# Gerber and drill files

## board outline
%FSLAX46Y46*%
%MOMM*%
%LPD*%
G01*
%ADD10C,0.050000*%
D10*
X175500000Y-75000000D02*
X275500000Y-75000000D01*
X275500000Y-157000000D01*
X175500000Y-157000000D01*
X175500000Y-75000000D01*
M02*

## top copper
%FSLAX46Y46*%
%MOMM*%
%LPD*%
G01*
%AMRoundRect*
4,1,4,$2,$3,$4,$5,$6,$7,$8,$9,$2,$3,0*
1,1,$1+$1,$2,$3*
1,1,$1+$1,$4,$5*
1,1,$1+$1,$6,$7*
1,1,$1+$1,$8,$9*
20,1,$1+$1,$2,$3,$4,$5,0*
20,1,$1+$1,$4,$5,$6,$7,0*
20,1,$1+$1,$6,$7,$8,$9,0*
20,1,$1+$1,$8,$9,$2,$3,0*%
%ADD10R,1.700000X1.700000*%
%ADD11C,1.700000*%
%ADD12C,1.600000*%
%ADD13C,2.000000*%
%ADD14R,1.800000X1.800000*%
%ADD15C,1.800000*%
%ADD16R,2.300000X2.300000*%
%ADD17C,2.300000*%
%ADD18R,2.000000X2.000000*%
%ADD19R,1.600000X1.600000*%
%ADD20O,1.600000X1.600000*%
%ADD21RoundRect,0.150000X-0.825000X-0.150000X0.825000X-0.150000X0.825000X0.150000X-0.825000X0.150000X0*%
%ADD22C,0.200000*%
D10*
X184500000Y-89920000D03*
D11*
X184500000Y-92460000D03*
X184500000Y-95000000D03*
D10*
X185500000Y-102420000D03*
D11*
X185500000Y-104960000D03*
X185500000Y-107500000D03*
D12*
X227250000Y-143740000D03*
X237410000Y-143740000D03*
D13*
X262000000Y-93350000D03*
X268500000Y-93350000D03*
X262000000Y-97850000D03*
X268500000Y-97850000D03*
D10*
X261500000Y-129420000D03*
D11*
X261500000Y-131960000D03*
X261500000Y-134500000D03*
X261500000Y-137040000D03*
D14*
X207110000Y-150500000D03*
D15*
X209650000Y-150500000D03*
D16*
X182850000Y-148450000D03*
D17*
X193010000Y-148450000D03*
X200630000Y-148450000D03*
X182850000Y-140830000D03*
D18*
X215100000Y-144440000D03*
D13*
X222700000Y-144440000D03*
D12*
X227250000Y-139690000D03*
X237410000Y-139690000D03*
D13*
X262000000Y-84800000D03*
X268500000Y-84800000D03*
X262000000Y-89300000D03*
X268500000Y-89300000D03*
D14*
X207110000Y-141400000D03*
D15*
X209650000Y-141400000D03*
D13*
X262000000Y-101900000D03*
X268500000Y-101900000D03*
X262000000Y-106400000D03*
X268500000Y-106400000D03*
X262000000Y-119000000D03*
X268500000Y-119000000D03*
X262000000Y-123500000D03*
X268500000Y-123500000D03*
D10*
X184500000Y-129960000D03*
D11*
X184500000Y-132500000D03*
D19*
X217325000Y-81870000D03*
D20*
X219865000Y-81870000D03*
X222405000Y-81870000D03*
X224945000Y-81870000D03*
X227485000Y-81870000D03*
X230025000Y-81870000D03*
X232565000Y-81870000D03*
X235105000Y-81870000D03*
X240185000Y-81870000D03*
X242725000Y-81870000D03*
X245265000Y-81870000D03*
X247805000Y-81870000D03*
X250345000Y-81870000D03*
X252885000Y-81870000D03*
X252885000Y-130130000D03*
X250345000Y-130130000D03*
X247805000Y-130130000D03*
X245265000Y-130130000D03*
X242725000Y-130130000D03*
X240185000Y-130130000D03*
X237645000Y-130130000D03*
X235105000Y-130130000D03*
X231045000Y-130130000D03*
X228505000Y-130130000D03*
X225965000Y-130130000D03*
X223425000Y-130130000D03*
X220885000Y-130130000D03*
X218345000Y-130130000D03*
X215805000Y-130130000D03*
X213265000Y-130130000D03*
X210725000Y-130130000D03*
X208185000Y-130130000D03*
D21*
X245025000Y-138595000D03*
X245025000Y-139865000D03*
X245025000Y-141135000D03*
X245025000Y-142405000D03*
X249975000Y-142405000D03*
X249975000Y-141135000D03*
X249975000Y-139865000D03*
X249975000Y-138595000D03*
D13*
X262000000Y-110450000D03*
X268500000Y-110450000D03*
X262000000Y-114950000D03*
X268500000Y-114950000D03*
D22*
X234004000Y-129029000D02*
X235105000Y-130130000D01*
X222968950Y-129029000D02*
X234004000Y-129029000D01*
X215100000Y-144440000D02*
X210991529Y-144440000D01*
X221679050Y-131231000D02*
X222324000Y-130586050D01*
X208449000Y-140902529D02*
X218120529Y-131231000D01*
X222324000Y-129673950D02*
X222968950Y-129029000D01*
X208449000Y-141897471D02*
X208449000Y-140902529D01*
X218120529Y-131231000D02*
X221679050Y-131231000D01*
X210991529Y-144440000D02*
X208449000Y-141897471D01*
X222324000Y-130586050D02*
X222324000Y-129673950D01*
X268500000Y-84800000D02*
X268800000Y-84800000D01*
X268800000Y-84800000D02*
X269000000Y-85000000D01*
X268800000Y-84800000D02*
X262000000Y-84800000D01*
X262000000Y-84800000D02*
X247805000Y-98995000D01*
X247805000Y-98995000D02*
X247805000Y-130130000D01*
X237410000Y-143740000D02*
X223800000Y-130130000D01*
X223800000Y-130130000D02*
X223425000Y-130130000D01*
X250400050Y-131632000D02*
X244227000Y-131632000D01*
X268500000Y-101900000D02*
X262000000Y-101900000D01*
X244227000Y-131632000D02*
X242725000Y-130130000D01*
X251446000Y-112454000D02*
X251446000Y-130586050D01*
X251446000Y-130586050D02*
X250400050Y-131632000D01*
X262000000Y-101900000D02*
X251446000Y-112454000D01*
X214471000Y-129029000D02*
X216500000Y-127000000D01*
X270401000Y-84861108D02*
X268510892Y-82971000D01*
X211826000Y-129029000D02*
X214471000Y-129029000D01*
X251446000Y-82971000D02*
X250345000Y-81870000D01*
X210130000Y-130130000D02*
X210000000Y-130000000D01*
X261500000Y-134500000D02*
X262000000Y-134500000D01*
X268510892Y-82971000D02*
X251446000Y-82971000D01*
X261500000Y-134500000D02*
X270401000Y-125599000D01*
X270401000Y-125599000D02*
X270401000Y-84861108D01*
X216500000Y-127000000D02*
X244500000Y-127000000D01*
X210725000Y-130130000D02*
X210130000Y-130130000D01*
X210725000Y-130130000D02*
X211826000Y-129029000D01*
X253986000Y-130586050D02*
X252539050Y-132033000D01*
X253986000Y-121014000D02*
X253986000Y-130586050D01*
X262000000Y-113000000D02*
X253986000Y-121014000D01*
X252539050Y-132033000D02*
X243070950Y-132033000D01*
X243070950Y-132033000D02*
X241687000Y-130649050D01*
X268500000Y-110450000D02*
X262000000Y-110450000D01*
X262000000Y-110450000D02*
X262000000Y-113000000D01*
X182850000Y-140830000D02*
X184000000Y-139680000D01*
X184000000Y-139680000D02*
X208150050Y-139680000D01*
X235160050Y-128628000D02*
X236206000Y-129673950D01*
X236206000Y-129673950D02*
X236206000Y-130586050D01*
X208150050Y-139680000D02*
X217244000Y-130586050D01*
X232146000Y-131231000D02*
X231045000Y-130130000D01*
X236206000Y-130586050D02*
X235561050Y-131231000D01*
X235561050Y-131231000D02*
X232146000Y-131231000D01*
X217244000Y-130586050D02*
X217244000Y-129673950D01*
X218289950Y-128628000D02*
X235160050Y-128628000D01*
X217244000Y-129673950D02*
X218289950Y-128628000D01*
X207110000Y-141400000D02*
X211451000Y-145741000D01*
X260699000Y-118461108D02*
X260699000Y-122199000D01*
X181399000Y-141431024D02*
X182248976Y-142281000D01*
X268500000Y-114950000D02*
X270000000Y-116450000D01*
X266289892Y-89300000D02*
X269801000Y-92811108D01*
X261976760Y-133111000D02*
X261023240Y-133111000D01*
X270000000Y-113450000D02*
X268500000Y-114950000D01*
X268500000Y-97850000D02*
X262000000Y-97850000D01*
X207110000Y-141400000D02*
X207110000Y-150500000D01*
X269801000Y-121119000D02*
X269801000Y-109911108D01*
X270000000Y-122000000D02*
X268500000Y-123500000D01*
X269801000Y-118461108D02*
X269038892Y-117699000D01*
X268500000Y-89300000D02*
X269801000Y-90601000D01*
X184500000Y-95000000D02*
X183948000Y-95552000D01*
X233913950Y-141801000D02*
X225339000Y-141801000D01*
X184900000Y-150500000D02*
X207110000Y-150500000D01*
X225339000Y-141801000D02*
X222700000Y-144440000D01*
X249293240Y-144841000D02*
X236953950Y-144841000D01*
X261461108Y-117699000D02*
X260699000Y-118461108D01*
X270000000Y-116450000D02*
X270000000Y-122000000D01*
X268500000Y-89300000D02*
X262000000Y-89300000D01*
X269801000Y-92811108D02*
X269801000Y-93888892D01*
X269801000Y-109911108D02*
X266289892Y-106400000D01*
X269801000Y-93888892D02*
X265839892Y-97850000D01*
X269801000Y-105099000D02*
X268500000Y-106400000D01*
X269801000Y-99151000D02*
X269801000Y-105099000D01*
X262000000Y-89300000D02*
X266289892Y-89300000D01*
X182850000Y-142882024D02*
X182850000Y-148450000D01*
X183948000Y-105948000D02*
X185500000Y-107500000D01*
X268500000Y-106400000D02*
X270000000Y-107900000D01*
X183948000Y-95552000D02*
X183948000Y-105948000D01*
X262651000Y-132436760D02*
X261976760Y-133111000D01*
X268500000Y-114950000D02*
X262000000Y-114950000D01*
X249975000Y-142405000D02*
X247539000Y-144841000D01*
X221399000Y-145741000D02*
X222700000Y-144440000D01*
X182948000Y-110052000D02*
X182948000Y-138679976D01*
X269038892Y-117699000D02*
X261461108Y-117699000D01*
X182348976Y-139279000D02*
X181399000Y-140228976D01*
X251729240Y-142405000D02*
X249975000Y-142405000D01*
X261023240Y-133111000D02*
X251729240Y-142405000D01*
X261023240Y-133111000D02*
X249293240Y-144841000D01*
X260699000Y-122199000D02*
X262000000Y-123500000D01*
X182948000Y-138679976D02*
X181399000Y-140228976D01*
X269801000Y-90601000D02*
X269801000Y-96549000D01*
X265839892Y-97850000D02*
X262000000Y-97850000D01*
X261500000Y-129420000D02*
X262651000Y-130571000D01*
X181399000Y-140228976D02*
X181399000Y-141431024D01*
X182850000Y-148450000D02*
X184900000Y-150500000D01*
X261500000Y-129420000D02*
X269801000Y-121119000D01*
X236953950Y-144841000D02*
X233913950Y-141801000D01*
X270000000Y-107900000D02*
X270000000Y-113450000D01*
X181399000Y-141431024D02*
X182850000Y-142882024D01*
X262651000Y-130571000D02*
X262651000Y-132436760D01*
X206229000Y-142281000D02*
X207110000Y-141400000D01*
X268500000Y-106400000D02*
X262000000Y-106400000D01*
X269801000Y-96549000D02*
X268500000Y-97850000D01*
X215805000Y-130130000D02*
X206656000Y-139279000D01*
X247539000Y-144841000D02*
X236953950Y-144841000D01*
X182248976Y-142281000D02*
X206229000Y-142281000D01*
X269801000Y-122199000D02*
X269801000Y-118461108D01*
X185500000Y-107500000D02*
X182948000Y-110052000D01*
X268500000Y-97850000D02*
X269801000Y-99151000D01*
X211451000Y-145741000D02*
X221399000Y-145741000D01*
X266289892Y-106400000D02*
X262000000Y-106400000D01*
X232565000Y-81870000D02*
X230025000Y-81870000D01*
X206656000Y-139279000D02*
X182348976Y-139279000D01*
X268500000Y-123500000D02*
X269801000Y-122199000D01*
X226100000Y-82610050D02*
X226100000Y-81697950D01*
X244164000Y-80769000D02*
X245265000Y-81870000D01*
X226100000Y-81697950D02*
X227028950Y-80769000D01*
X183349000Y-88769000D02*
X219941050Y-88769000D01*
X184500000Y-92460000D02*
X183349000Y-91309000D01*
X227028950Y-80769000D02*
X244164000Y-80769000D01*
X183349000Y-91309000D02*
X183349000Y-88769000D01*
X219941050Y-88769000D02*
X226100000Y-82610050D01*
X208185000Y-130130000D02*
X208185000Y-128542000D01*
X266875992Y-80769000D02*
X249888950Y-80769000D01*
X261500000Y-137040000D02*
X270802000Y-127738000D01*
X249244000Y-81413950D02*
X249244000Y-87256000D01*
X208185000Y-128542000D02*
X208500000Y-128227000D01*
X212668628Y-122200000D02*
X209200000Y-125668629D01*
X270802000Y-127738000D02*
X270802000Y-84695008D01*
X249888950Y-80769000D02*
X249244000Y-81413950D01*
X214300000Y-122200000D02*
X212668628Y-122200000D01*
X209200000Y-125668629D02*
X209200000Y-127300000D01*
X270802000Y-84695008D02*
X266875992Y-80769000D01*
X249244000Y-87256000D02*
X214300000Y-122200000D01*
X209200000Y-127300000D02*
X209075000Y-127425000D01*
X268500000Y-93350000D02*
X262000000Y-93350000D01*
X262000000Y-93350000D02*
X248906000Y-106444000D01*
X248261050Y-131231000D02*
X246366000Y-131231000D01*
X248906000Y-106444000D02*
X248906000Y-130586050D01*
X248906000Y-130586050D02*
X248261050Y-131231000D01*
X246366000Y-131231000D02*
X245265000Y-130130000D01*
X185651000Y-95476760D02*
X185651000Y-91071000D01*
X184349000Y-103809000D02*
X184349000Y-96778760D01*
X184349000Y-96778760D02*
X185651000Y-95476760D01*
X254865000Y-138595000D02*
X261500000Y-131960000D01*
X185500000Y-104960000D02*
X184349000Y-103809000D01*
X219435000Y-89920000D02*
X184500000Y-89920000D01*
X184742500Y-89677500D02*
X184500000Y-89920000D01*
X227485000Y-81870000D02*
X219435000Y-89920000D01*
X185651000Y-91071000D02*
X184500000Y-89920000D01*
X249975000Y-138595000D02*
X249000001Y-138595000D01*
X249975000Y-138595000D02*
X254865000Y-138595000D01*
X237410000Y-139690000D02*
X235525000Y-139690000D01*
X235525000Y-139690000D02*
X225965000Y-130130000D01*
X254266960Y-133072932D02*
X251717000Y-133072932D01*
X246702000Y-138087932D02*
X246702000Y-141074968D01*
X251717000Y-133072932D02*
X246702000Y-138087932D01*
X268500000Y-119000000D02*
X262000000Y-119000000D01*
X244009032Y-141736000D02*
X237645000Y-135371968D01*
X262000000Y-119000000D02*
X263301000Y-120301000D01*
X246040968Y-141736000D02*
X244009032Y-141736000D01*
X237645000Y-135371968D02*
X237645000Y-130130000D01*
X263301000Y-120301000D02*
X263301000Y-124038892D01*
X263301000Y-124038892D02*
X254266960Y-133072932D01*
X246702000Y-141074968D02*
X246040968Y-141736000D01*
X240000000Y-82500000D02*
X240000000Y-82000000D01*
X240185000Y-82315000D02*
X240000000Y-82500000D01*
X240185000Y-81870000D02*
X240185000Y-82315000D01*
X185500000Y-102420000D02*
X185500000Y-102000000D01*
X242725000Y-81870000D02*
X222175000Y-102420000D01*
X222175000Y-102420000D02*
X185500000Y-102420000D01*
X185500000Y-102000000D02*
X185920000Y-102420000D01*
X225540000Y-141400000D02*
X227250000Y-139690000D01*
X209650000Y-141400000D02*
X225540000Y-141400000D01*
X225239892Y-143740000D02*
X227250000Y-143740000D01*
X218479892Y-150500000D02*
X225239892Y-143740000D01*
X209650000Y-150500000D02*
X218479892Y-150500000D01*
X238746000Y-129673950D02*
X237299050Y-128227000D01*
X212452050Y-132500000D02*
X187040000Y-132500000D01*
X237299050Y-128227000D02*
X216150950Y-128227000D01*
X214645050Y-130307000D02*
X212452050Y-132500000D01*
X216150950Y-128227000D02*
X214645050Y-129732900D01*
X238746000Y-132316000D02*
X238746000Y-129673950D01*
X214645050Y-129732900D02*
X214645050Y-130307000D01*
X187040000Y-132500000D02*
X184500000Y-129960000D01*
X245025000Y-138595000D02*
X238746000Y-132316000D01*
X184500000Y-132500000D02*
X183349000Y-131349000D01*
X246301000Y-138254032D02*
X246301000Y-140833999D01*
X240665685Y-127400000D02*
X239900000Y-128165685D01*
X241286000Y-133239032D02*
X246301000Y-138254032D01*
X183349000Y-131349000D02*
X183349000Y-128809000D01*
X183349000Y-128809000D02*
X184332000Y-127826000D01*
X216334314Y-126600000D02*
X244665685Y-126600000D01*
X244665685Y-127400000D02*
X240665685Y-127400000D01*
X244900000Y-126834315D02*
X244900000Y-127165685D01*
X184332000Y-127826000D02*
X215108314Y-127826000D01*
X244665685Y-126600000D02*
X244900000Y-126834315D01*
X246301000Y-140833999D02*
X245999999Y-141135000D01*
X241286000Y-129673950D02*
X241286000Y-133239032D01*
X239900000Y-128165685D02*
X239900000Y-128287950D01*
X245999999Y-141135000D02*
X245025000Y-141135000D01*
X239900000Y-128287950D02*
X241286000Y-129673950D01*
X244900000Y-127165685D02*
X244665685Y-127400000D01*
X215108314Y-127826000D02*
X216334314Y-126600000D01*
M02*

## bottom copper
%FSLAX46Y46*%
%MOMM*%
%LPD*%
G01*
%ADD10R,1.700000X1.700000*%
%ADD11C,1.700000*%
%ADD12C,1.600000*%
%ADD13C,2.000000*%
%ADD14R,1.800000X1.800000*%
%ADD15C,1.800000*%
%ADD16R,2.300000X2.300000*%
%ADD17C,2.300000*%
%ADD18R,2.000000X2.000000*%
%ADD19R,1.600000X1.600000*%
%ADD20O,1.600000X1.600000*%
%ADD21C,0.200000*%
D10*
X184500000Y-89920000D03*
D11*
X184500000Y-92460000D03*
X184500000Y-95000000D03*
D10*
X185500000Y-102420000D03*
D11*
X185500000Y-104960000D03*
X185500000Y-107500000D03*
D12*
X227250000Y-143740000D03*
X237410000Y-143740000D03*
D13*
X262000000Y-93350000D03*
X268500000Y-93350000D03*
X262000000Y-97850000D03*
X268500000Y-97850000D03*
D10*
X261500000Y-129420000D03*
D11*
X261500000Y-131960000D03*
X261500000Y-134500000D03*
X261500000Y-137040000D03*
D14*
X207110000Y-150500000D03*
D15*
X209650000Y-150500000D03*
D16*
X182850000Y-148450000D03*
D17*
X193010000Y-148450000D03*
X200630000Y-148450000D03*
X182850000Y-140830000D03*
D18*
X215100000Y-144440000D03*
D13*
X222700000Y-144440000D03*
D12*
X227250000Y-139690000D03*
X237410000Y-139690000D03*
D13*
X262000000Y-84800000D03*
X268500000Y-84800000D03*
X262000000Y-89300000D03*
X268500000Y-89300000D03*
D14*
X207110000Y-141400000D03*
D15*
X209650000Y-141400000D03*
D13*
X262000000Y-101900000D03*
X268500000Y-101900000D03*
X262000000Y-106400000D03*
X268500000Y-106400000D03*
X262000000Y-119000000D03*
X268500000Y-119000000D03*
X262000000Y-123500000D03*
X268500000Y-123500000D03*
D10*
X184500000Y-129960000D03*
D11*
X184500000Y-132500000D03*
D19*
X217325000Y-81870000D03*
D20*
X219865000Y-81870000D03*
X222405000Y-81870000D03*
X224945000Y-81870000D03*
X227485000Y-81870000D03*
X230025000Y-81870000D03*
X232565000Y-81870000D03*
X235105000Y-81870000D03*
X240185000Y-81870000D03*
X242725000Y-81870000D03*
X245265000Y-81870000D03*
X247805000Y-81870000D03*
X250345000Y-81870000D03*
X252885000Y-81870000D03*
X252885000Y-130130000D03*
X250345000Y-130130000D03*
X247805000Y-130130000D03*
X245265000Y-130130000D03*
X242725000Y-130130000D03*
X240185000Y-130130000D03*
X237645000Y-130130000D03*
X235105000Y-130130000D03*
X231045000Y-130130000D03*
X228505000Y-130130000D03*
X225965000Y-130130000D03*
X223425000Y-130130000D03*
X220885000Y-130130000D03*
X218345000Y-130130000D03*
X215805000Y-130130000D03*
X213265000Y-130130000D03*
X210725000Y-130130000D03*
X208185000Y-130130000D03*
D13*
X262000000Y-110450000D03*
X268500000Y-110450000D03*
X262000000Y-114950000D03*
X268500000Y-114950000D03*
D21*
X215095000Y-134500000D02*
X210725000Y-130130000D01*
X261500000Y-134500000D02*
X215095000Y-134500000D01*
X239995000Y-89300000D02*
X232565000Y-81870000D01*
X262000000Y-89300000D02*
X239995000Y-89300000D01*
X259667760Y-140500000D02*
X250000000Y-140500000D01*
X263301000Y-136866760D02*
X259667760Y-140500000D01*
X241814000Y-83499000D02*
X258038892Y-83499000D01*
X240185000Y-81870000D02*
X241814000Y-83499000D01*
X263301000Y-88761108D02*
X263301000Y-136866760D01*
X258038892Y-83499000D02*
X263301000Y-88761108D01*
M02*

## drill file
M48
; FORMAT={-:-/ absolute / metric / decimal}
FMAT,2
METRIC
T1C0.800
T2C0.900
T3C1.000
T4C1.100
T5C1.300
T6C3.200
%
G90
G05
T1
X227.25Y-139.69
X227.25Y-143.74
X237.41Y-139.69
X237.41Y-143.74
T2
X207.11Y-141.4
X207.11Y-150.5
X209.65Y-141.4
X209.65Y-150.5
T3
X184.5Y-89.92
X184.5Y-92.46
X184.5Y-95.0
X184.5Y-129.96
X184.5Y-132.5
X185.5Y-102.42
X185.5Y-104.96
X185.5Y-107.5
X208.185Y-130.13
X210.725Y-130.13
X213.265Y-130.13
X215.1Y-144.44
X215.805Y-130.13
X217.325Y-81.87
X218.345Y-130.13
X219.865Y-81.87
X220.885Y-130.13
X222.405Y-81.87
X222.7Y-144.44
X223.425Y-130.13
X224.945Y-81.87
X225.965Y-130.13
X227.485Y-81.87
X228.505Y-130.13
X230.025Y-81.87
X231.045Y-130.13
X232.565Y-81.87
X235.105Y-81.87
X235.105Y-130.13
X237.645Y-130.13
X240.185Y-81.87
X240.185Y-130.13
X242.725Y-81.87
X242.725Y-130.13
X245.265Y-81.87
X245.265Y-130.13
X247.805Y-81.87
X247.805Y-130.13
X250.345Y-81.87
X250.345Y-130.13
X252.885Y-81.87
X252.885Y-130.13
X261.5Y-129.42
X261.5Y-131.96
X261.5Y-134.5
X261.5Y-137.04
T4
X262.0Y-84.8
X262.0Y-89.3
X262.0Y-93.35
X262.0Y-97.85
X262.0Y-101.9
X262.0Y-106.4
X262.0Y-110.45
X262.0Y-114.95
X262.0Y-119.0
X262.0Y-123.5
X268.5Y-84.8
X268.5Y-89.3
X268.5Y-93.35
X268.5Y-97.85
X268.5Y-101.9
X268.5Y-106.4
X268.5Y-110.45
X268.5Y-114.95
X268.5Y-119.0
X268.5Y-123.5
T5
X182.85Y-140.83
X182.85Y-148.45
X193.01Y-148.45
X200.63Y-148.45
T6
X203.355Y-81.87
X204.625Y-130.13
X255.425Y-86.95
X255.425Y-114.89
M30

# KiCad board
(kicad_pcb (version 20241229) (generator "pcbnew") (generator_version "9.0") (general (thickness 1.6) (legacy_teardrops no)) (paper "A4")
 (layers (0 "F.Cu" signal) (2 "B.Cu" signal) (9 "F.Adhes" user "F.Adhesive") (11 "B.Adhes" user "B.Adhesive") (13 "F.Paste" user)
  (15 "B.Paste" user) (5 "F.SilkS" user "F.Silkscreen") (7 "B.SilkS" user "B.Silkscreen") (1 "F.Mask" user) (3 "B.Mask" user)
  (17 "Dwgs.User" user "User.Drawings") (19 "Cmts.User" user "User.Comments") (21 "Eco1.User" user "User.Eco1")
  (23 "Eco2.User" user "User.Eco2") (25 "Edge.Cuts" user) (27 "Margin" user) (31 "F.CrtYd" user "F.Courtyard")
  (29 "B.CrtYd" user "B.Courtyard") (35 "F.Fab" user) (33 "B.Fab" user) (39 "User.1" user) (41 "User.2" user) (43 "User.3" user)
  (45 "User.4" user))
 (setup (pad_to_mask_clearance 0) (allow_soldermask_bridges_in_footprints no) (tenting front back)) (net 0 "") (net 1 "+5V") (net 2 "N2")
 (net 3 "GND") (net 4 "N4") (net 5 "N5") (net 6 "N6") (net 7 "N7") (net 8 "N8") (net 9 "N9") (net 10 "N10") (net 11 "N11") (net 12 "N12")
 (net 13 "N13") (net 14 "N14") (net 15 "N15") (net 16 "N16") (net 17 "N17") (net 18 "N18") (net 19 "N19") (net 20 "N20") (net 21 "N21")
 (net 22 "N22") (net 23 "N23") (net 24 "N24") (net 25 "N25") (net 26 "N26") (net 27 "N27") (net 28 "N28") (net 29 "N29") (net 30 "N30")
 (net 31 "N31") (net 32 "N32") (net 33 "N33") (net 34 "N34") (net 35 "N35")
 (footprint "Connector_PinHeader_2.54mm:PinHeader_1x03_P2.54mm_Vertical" (layer "F.Cu") (at 184.5 89.92)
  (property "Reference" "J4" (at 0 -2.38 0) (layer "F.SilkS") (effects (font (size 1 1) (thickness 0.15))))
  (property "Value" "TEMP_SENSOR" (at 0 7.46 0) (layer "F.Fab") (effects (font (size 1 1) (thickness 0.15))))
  (pad "1" thru_hole rect (at 0 0) (size 1.7 1.7) (drill 1) (layers "*.Cu" "*.Mask") (remove_unused_layers no) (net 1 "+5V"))
  (pad "2" thru_hole circle (at 0 2.54) (size 1.7 1.7) (drill 1) (layers "*.Cu" "*.Mask") (remove_unused_layers no) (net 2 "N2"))
  (pad "3" thru_hole circle (at 0 5.08) (size 1.7 1.7) (drill 1) (layers "*.Cu" "*.Mask") (remove_unused_layers no) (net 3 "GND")))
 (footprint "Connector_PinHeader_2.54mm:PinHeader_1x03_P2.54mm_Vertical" (layer "F.Cu") (at 185.5 102.42)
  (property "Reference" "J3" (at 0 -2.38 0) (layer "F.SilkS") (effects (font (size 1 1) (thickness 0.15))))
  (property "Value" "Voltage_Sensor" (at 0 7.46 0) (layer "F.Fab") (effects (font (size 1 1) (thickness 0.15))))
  (pad "1" thru_hole rect (at 0 0) (size 1.7 1.7) (drill 1) (layers "*.Cu" "*.Mask") (remove_unused_layers no) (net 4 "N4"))
  (pad "2" thru_hole circle (at 0 2.54) (size 1.7 1.7) (drill 1) (layers "*.Cu" "*.Mask") (remove_unused_layers no) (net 1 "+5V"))
  (pad "3" thru_hole circle (at 0 5.08) (size 1.7 1.7) (drill 1) (layers "*.Cu" "*.Mask") (remove_unused_layers no) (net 3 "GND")))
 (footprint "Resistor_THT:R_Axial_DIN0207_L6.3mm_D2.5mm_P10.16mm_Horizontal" (layer "F.Cu") (at 227.25 143.74)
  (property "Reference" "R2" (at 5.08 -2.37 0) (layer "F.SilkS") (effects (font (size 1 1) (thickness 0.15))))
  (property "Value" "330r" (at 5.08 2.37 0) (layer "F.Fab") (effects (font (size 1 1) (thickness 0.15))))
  (pad "1" thru_hole circle (at 0 0) (size 1.6 1.6) (drill 0.8) (layers "*.Cu" "*.Mask") (remove_unused_layers no) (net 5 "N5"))
  (pad "2" thru_hole circle (at 10.16 0) (size 1.6 1.6) (drill 0.8) (layers "*.Cu" "*.Mask") (remove_unused_layers no) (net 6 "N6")))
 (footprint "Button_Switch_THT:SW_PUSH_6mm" (layer "F.Cu") (at 262 93.35)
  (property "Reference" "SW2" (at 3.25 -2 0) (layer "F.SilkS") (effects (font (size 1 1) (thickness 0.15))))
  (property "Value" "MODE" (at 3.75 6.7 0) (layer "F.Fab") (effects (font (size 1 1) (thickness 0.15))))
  (pad "1" thru_hole circle (at 0 0 90) (size 2 2) (drill 1.1) (layers "*.Cu" "*.Mask") (remove_unused_layers no) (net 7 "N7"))
  (pad "1" thru_hole circle (at 6.5 0 90) (size 2 2) (drill 1.1) (layers "*.Cu" "*.Mask") (remove_unused_layers no) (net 7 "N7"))
  (pad "2" thru_hole circle (at 0 4.5 90) (size 2 2) (drill 1.1) (layers "*.Cu" "*.Mask") (remove_unused_layers no) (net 3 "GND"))
  (pad "2" thru_hole circle (at 6.5 4.5 90) (size 2 2) (drill 1.1) (layers "*.Cu" "*.Mask") (remove_unused_layers no) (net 3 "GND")))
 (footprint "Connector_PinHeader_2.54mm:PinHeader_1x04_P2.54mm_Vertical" (layer "F.Cu") (at 261.5 129.42)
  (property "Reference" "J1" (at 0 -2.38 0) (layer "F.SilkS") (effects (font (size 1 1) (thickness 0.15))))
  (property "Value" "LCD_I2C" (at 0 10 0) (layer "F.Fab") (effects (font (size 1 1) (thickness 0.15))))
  (pad "1" thru_hole rect (at 0 0) (size 1.7 1.7) (drill 1) (layers "*.Cu" "*.Mask") (remove_unused_layers no) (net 3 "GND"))
  (pad "2" thru_hole circle (at 0 2.54) (size 1.7 1.7) (drill 1) (layers "*.Cu" "*.Mask") (remove_unused_layers no) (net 1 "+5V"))
  (pad "3" thru_hole circle (at 0 5.08) (size 1.7 1.7) (drill 1) (layers "*.Cu" "*.Mask") (remove_unused_layers no) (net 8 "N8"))
  (pad "4" thru_hole circle (at 0 7.62) (size 1.7 1.7) (drill 1) (layers "*.Cu" "*.Mask") (remove_unused_layers no) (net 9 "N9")))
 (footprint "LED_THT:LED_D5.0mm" (layer "F.Cu") (at 207.11 150.5)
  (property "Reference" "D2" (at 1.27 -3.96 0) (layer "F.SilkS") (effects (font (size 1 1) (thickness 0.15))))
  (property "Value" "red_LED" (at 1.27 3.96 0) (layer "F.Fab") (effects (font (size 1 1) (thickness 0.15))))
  (pad "1" thru_hole rect (at 0 0) (size 1.8 1.8) (drill 0.9) (layers "*.Cu" "*.Mask") (remove_unused_layers no) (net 3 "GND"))
  (pad "2" thru_hole circle (at 2.54 0) (size 1.8 1.8) (drill 0.9) (layers "*.Cu" "*.Mask") (remove_unused_layers no) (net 5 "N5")))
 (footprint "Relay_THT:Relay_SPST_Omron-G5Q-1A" (layer "F.Cu") (at 182.85 148.45)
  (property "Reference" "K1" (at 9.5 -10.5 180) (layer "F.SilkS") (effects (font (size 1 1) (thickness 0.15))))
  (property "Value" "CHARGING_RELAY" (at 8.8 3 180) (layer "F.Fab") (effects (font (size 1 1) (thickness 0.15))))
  (pad "1" thru_hole rect (at 0 0 180) (size 2.3 2.3) (drill 1.3) (layers "*.Cu" "*.Mask") (remove_unused_layers no) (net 3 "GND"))
  (pad "2" thru_hole circle (at 10.16 0 180) (size 2.3 2.3) (drill 1.3) (layers "*.Cu" "*.Mask") (remove_unused_layers no) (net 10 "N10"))
  (pad "3" thru_hole circle (at 17.78 0 180) (size 2.3 2.3) (drill 1.3) (layers "*.Cu" "*.Mask") (remove_unused_layers no) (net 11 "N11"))
  (pad "5" thru_hole circle (at 0 -7.62 180) (size 2.3 2.3) (drill 1.3) (layers "*.Cu" "*.Mask") (remove_unused_layers no) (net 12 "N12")))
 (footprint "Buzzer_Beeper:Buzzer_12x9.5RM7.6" (layer "F.Cu") (at 215.1 144.44)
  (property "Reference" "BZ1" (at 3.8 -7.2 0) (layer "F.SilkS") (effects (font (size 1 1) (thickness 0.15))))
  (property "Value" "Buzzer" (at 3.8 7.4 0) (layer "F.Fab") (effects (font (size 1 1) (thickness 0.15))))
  (pad "1" thru_hole rect (at 0 0) (size 2 2) (drill 1) (layers "*.Cu" "*.Mask") (remove_unused_layers no) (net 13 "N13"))
  (pad "2" thru_hole circle (at 7.6 0) (size 2 2) (drill 1) (layers "*.Cu" "*.Mask") (remove_unused_layers no) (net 3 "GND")))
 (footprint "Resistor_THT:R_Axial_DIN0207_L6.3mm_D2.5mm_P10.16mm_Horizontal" (layer "F.Cu") (at 227.25 139.69)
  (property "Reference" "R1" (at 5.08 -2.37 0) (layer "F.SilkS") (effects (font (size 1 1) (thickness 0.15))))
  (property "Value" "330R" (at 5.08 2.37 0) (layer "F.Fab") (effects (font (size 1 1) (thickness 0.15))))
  (pad "1" thru_hole circle (at 0 0) (size 1.6 1.6) (drill 0.8) (layers "*.Cu" "*.Mask") (remove_unused_layers no) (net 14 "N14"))
  (pad "2" thru_hole circle (at 10.16 0) (size 1.6 1.6) (drill 0.8) (layers "*.Cu" "*.Mask") (remove_unused_layers no) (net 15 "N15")))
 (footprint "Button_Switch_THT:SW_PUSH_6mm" (layer "F.Cu") (at 262 84.8)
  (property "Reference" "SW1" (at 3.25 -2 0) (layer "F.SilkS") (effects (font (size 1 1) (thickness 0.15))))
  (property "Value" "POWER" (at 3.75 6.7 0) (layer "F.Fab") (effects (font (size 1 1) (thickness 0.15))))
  (pad "1" thru_hole circle (at 0 0 90) (size 2 2) (drill 1.1) (layers "*.Cu" "*.Mask") (remove_unused_layers no) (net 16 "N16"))
  (pad "1" thru_hole circle (at 6.5 0 90) (size 2 2) (drill 1.1) (layers "*.Cu" "*.Mask") (remove_unused_layers no) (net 16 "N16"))
  (pad "2" thru_hole circle (at 0 4.5 90) (size 2 2) (drill 1.1) (layers "*.Cu" "*.Mask") (remove_unused_layers no) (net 3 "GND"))
  (pad "2" thru_hole circle (at 6.5 4.5 90) (size 2 2) (drill 1.1) (layers "*.Cu" "*.Mask") (remove_unused_layers no) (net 3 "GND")))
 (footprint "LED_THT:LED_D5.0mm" (layer "F.Cu") (at 207.11 141.4)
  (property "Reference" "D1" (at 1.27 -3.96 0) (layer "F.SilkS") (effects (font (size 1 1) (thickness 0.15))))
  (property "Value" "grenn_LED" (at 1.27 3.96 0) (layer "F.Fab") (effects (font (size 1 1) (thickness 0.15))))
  (pad "1" thru_hole rect (at 0 0) (size 1.8 1.8) (drill 0.9) (layers "*.Cu" "*.Mask") (remove_unused_layers no) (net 3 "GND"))
  (pad "2" thru_hole circle (at 2.54 0) (size 1.8 1.8) (drill 0.9) (layers "*.Cu" "*.Mask") (remove_unused_layers no) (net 14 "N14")))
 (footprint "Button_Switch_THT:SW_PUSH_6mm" (layer "F.Cu") (at 262 101.9)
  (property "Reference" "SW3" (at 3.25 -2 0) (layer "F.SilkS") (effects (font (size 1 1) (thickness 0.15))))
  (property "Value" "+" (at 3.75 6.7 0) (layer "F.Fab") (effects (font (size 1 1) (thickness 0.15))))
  (pad "1" thru_hole circle (at 0 0 90) (size 2 2) (drill 1.1) (layers "*.Cu" "*.Mask") (remove_unused_layers no) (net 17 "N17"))
  (pad "1" thru_hole circle (at 6.5 0 90) (size 2 2) (drill 1.1) (layers "*.Cu" "*.Mask") (remove_unused_layers no) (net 17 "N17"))
  (pad "2" thru_hole circle (at 0 4.5 90) (size 2 2) (drill 1.1) (layers "*.Cu" "*.Mask") (remove_unused_layers no) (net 3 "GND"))
  (pad "2" thru_hole circle (at 6.5 4.5 90) (size 2 2) (drill 1.1) (layers "*.Cu" "*.Mask") (remove_unused_layers no) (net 3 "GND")))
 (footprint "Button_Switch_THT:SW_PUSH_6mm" (layer "F.Cu") (at 262 119)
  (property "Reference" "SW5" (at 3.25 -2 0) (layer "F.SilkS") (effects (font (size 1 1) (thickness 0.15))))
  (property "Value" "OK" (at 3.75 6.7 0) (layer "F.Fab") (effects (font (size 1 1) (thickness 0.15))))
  (pad "1" thru_hole circle (at 0 0 90) (size 2 2) (drill 1.1) (layers "*.Cu" "*.Mask") (remove_unused_layers no) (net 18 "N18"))
  (pad "1" thru_hole circle (at 6.5 0 90) (size 2 2) (drill 1.1) (layers "*.Cu" "*.Mask") (remove_unused_layers no) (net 18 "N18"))
  (pad "2" thru_hole circle (at 0 4.5 90) (size 2 2) (drill 1.1) (layers "*.Cu" "*.Mask") (remove_unused_layers no) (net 3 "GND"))
  (pad "2" thru_hole circle (at 6.5 4.5 90) (size 2 2) (drill 1.1) (layers "*.Cu" "*.Mask") (remove_unused_layers no) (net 3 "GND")))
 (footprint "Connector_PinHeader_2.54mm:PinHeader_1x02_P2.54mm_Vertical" (layer "F.Cu") (at 184.5 129.96)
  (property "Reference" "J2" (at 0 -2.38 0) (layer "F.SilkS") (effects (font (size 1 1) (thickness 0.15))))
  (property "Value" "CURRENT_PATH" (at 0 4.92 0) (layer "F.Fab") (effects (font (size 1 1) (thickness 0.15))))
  (pad "1" thru_hole rect (at 0 0) (size 1.7 1.7) (drill 1) (layers "*.Cu" "*.Mask") (remove_unused_layers no) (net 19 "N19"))
  (pad "2" thru_hole circle (at 0 2.54) (size 1.7 1.7) (drill 1) (layers "*.Cu" "*.Mask") (remove_unused_layers no) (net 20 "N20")))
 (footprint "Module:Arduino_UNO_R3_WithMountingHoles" (layer "F.Cu") (at 217.325 81.87)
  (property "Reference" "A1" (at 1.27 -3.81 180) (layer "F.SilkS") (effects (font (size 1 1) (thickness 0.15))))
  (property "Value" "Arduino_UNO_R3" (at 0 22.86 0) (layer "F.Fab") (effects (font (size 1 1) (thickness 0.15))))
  (pad "" np_thru_hole circle (at -13.97 0 90) (size 3.2 3.2) (drill 3.2) (layers "*.Cu" "*.Mask"))
  (pad "" np_thru_hole circle (at -12.7 48.26 90) (size 3.2 3.2) (drill 3.2) (layers "*.Cu" "*.Mask"))
  (pad "" np_thru_hole circle (at 38.1 5.08 90) (size 3.2 3.2) (drill 3.2) (layers "*.Cu" "*.Mask"))
  (pad "" np_thru_hole circle (at 38.1 33.02 90) (size 3.2 3.2) (drill 3.2) (layers "*.Cu" "*.Mask"))
  (pad "1" thru_hole rect (at 0 0 90) (size 1.6 1.6) (drill 1) (layers "*.Cu" "*.Mask") (remove_unused_layers no) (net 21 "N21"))
  (pad "2" thru_hole oval (at 2.54 0 90) (size 1.6 1.6) (drill 1) (layers "*.Cu" "*.Mask") (remove_unused_layers no) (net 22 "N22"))
  (pad "3" thru_hole oval (at 5.08 0 90) (size 1.6 1.6) (drill 1) (layers "*.Cu" "*.Mask") (remove_unused_layers no) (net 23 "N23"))
  (pad "4" thru_hole oval (at 7.62 0 90) (size 1.6 1.6) (drill 1) (layers "*.Cu" "*.Mask") (remove_unused_layers no) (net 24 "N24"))
  (pad "5" thru_hole oval (at 10.16 0 90) (size 1.6 1.6) (drill 1) (layers "*.Cu" "*.Mask") (remove_unused_layers no) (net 1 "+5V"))
  (pad "6" thru_hole oval (at 12.7 0 90) (size 1.6 1.6) (drill 1) (layers "*.Cu" "*.Mask") (remove_unused_layers no) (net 3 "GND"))
  (pad "7" thru_hole oval (at 15.24 0 90) (size 1.6 1.6) (drill 1) (layers "*.Cu" "*.Mask") (remove_unused_layers no) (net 3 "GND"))
  (pad "8" thru_hole oval (at 17.78 0 90) (size 1.6 1.6) (drill 1) (layers "*.Cu" "*.Mask") (remove_unused_layers no) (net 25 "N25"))
  (pad "9" thru_hole oval (at 22.86 0 90) (size 1.6 1.6) (drill 1) (layers "*.Cu" "*.Mask") (remove_unused_layers no) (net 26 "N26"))
  (pad "10" thru_hole oval (at 25.4 0 90) (size 1.6 1.6) (drill 1) (layers "*.Cu" "*.Mask") (remove_unused_layers no) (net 4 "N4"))
  (pad "11" thru_hole oval (at 27.94 0 90) (size 1.6 1.6) (drill 1) (layers "*.Cu" "*.Mask") (remove_unused_layers no) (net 2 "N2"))
  (pad "12" thru_hole oval (at 30.48 0 90) (size 1.6 1.6) (drill 1) (layers "*.Cu" "*.Mask") (remove_unused_layers no) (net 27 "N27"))
  (pad "13" thru_hole oval (at 33.02 0 90) (size 1.6 1.6) (drill 1) (layers "*.Cu" "*.Mask") (remove_unused_layers no) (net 8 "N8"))
  (pad "14" thru_hole oval (at 35.56 0 90) (size 1.6 1.6) (drill 1) (layers "*.Cu" "*.Mask") (remove_unused_layers no) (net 9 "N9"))
  (pad "15" thru_hole oval (at 35.56 48.26 90) (size 1.6 1.6) (drill 1) (layers "*.Cu" "*.Mask") (remove_unused_layers no) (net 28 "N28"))
  (pad "16" thru_hole oval (at 33.02 48.26 90) (size 1.6 1.6) (drill 1) (layers "*.Cu" "*.Mask") (remove_unused_layers no) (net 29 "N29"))
  (pad "17" thru_hole oval (at 30.48 48.26 90) (size 1.6 1.6) (drill 1) (layers "*.Cu" "*.Mask") (remove_unused_layers no) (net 16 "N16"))
  (pad "18" thru_hole oval (at 27.94 48.26 90) (size 1.6 1.6) (drill 1) (layers "*.Cu" "*.Mask") (remove_unused_layers no) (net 7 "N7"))
  (pad "19" thru_hole oval (at 25.4 48.26 90) (size 1.6 1.6) (drill 1) (layers "*.Cu" "*.Mask") (remove_unused_layers no) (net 17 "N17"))
  (pad "20" thru_hole oval (at 22.86 48.26 90) (size 1.6 1.6) (drill 1) (layers "*.Cu" "*.Mask") (remove_unused_layers no) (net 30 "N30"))
  (pad "21" thru_hole oval (at 20.32 48.26 90) (size 1.6 1.6) (drill 1) (layers "*.Cu" "*.Mask") (remove_unused_layers no) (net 18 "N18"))
  (pad "22" thru_hole oval (at 17.78 48.26 90) (size 1.6 1.6) (drill 1) (layers "*.Cu" "*.Mask") (remove_unused_layers no) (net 13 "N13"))
  (pad "23" thru_hole oval (at 13.72 48.26 90) (size 1.6 1.6) (drill 1) (layers "*.Cu" "*.Mask") (remove_unused_layers no) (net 12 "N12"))
  (pad "24" thru_hole oval (at 11.18 48.26 90) (size 1.6 1.6) (drill 1) (layers "*.Cu" "*.Mask") (remove_unused_layers no) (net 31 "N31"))
  (pad "25" thru_hole oval (at 8.64 48.26 90) (size 1.6 1.6) (drill 1) (layers "*.Cu" "*.Mask") (remove_unused_layers no) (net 15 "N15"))
  (pad "26" thru_hole oval (at 6.1 48.26 90) (size 1.6 1.6) (drill 1) (layers "*.Cu" "*.Mask") (remove_unused_layers no) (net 6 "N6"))
  (pad "27" thru_hole oval (at 3.56 48.26 90) (size 1.6 1.6) (drill 1) (layers "*.Cu" "*.Mask") (remove_unused_layers no) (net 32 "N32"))
  (pad "28" thru_hole oval (at 1.02 48.26 90) (size 1.6 1.6) (drill 1) (layers "*.Cu" "*.Mask") (remove_unused_layers no) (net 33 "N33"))
  (pad "29" thru_hole oval (at -1.52 48.26 90) (size 1.6 1.6) (drill 1) (layers "*.Cu" "*.Mask") (remove_unused_layers no) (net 3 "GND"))
  (pad "30" thru_hole oval (at -4.06 48.26 90) (size 1.6 1.6) (drill 1) (layers "*.Cu" "*.Mask") (remove_unused_layers no) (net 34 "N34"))
  (pad "31" thru_hole oval (at -6.6 48.26 90) (size 1.6 1.6) (drill 1) (layers "*.Cu" "*.Mask") (remove_unused_layers no) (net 8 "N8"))
  (pad "32" thru_hole oval (at -9.14 48.26 90) (size 1.6 1.6) (drill 1) (layers "*.Cu" "*.Mask") (remove_unused_layers no) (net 9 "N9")))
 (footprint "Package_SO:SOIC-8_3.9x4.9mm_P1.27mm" (layer "F.Cu") (at 247.5 140.5)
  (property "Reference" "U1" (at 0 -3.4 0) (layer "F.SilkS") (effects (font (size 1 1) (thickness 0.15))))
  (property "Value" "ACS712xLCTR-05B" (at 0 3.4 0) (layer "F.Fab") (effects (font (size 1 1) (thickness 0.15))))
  (pad "1" smd roundrect (at -2.475 -1.905) (size 1.95 0.6) (layers "F.Cu" "F.Mask" "F.Paste") (roundrect_rratio 0.25) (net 19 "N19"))
  (pad "2" smd roundrect (at -2.475 -0.635) (size 1.95 0.6) (layers "F.Cu" "F.Mask" "F.Paste") (roundrect_rratio 0.25) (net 19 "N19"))
  (pad "3" smd roundrect (at -2.475 0.635) (size 1.95 0.6) (layers "F.Cu" "F.Mask" "F.Paste") (roundrect_rratio 0.25) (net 20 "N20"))
  (pad "4" smd roundrect (at -2.475 1.905) (size 1.95 0.6) (layers "F.Cu" "F.Mask" "F.Paste") (roundrect_rratio 0.25) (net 20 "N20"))
  (pad "5" smd roundrect (at 2.475 1.905) (size 1.95 0.6) (layers "F.Cu" "F.Mask" "F.Paste") (roundrect_rratio 0.25) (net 3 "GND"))
  (pad "6" smd roundrect (at 2.475 0.635) (size 1.95 0.6) (layers "F.Cu" "F.Mask" "F.Paste") (roundrect_rratio 0.25) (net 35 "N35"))
  (pad "7" smd roundrect (at 2.475 -0.635) (size 1.95 0.6) (layers "F.Cu" "F.Mask" "F.Paste") (roundrect_rratio 0.25) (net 26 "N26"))
  (pad "8" smd roundrect (at 2.475 -1.905) (size 1.95 0.6) (layers "F.Cu" "F.Mask" "F.Paste") (roundrect_rratio 0.25) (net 1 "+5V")))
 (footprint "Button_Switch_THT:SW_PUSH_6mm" (layer "F.Cu") (at 262 110.45)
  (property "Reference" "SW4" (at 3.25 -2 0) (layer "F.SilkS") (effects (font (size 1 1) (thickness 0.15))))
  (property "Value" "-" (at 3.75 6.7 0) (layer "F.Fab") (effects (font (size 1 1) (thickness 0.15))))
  (pad "1" thru_hole circle (at 0 0 90) (size 2 2) (drill 1.1) (layers "*.Cu" "*.Mask") (remove_unused_layers no) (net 30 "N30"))
  (pad "1" thru_hole circle (at 6.5 0 90) (size 2 2) (drill 1.1) (layers "*.Cu" "*.Mask") (remove_unused_layers no) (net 30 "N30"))
  (pad "2" thru_hole circle (at 0 4.5 90) (size 2 2) (drill 1.1) (layers "*.Cu" "*.Mask") (remove_unused_layers no) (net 3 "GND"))
  (pad "2" thru_hole circle (at 6.5 4.5 90) (size 2 2) (drill 1.1) (layers "*.Cu" "*.Mask") (remove_unused_layers no) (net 3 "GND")))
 (gr_rect (start 175.5 75) (end 275.5 157) (stroke (width 0.05) (type default)) (fill no) (layer "Edge.Cuts"))
 (segment (start 234.004 129.029) (end 235.105 130.13) (width 0.2) (layer "F.Cu") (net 13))
 (segment (start 222.96895 129.029) (end 234.004 129.029) (width 0.2) (layer "F.Cu") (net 13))
 (segment (start 215.1 144.44) (end 210.991529 144.44) (width 0.2) (layer "F.Cu") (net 13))
 (segment (start 221.67905 131.231) (end 222.324 130.58605) (width 0.2) (layer "F.Cu") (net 13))
 (segment (start 208.449 140.902529) (end 218.120529 131.231) (width 0.2) (layer "F.Cu") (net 13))
 (segment (start 222.324 129.67395) (end 222.96895 129.029) (width 0.2) (layer "F.Cu") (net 13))
 (segment (start 208.449 141.897471) (end 208.449 140.902529) (width 0.2) (layer "F.Cu") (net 13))
 (segment (start 218.120529 131.231) (end 221.67905 131.231) (width 0.2) (layer "F.Cu") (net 13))
 (segment (start 210.991529 144.44) (end 208.449 141.897471) (width 0.2) (layer "F.Cu") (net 13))
 (segment (start 222.324 130.58605) (end 222.324 129.67395) (width 0.2) (layer "F.Cu") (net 13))
 (segment (start 268.5 84.8) (end 268.8 84.8) (width 0.2) (layer "F.Cu") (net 16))
 (segment (start 268.8 84.8) (end 269 85) (width 0.2) (layer "F.Cu") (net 16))
 (segment (start 268.8 84.8) (end 262 84.8) (width 0.2) (layer "F.Cu") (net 16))
 (segment (start 262 84.8) (end 247.805 98.995) (width 0.2) (layer "F.Cu") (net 16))
 (segment (start 247.805 98.995) (end 247.805 130.13) (width 0.2) (layer "F.Cu") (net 16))
 (segment (start 237.41 143.74) (end 223.8 130.13) (width 0.2) (layer "F.Cu") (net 6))
 (segment (start 223.8 130.13) (end 223.425 130.13) (width 0.2) (layer "F.Cu") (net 6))
 (segment (start 250.40005 131.632) (end 244.227 131.632) (width 0.2) (layer "F.Cu") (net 17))
 (segment (start 268.5 101.9) (end 262 101.9) (width 0.2) (layer "F.Cu") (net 17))
 (segment (start 244.227 131.632) (end 242.725 130.13) (width 0.2) (layer "F.Cu") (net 17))
 (segment (start 251.446 112.454) (end 251.446 130.58605) (width 0.2) (layer "F.Cu") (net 17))
 (segment (start 251.446 130.58605) (end 250.40005 131.632) (width 0.2) (layer "F.Cu") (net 17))
 (segment (start 262 101.9) (end 251.446 112.454) (width 0.2) (layer "F.Cu") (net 17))
 (segment (start 214.471 129.029) (end 216.5 127) (width 0.2) (layer "F.Cu") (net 8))
 (segment (start 270.401 84.861108) (end 268.510892 82.971) (width 0.2) (layer "F.Cu") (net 8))
 (segment (start 211.826 129.029) (end 214.471 129.029) (width 0.2) (layer "F.Cu") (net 8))
 (segment (start 251.446 82.971) (end 250.345 81.87) (width 0.2) (layer "F.Cu") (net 8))
 (segment (start 210.13 130.13) (end 210 130) (width 0.2) (layer "F.Cu") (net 8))
 (segment (start 261.5 134.5) (end 262 134.5) (width 0.2) (layer "F.Cu") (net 8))
 (segment (start 268.510892 82.971) (end 251.446 82.971) (width 0.2) (layer "F.Cu") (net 8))
 (segment (start 261.5 134.5) (end 270.401 125.599) (width 0.2) (layer "F.Cu") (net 8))
 (segment (start 270.401 125.599) (end 270.401 84.861108) (width 0.2) (layer "F.Cu") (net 8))
 (segment (start 216.5 127) (end 244.5 127) (width 0.2) (layer "F.Cu") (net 8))
 (segment (start 210.725 130.13) (end 210.13 130.13) (width 0.2) (layer "F.Cu") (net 8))
 (segment (start 210.725 130.13) (end 211.826 129.029) (width 0.2) (layer "F.Cu") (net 8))
 (segment (start 215.095 134.5) (end 210.725 130.13) (width 0.2) (layer "B.Cu") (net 8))
 (segment (start 261.5 134.5) (end 215.095 134.5) (width 0.2) (layer "B.Cu") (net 8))
 (segment (start 253.986 130.58605) (end 252.53905 132.033) (width 0.2) (layer "F.Cu") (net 30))
 (segment (start 253.986 121.014) (end 253.986 130.58605) (width 0.2) (layer "F.Cu") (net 30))
 (segment (start 262 113) (end 253.986 121.014) (width 0.2) (layer "F.Cu") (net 30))
 (segment (start 252.53905 132.033) (end 243.07095 132.033) (width 0.2) (layer "F.Cu") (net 30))
 (segment (start 243.07095 132.033) (end 241.687 130.64905) (width 0.2) (layer "F.Cu") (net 30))
 (segment (start 268.5 110.45) (end 262 110.45) (width 0.2) (layer "F.Cu") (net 30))
 (segment (start 262 110.45) (end 262 113) (width 0.2) (layer "F.Cu") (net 30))
 (segment (start 182.85 140.83) (end 184 139.68) (width 0.2) (layer "F.Cu") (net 12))
 (segment (start 184 139.68) (end 208.15005 139.68) (width 0.2) (layer "F.Cu") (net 12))
 (segment (start 235.16005 128.628) (end 236.206 129.67395) (width 0.2) (layer "F.Cu") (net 12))
 (segment (start 236.206 129.67395) (end 236.206 130.58605) (width 0.2) (layer "F.Cu") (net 12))
 (segment (start 208.15005 139.68) (end 217.244 130.58605) (width 0.2) (layer "F.Cu") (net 12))
 (segment (start 232.146 131.231) (end 231.045 130.13) (width 0.2) (layer "F.Cu") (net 12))
 (segment (start 236.206 130.58605) (end 235.56105 131.231) (width 0.2) (layer "F.Cu") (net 12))
 (segment (start 235.56105 131.231) (end 232.146 131.231) (width 0.2) (layer "F.Cu") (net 12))
 (segment (start 217.244 130.58605) (end 217.244 129.67395) (width 0.2) (layer "F.Cu") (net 12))
 (segment (start 218.28995 128.628) (end 235.16005 128.628) (width 0.2) (layer "F.Cu") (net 12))
 (segment (start 217.244 129.67395) (end 218.28995 128.628) (width 0.2) (layer "F.Cu") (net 12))
 (segment (start 207.11 141.4) (end 211.451 145.741) (width 0.2) (layer "F.Cu") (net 3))
 (segment (start 260.699 118.461108) (end 260.699 122.199) (width 0.2) (layer "F.Cu") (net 3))
 (segment (start 181.399 141.431024) (end 182.248976 142.281) (width 0.2) (layer "F.Cu") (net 3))
 (segment (start 268.5 114.95) (end 270 116.45) (width 0.2) (layer "F.Cu") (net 3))
 (segment (start 266.289892 89.3) (end 269.801 92.811108) (width 0.2) (layer "F.Cu") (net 3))
 (segment (start 261.97676 133.111) (end 261.02324 133.111) (width 0.2) (layer "F.Cu") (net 3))
 (segment (start 270 113.45) (end 268.5 114.95) (width 0.2) (layer "F.Cu") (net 3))
 (segment (start 268.5 97.85) (end 262 97.85) (width 0.2) (layer "F.Cu") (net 3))
 (segment (start 207.11 141.4) (end 207.11 150.5) (width 0.2) (layer "F.Cu") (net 3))
 (segment (start 269.801 121.119) (end 269.801 109.911108) (width 0.2) (layer "F.Cu") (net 3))
 (segment (start 270 122) (end 268.5 123.5) (width 0.2) (layer "F.Cu") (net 3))
 (segment (start 269.801 118.461108) (end 269.038892 117.699) (width 0.2) (layer "F.Cu") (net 3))
 (segment (start 268.5 89.3) (end 269.801 90.601) (width 0.2) (layer "F.Cu") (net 3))
 (segment (start 184.5 95) (end 183.948 95.552) (width 0.2) (layer "F.Cu") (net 3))
 (segment (start 233.91395 141.801) (end 225.339 141.801) (width 0.2) (layer "F.Cu") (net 3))
 (segment (start 184.9 150.5) (end 207.11 150.5) (width 0.2) (layer "F.Cu") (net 3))
 (segment (start 225.339 141.801) (end 222.7 144.44) (width 0.2) (layer "F.Cu") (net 3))
 (segment (start 249.29324 144.841) (end 236.95395 144.841) (width 0.2) (layer "F.Cu") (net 3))
 (segment (start 261.461108 117.699) (end 260.699 118.461108) (width 0.2) (layer "F.Cu") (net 3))
 (segment (start 270 116.45) (end 270 122) (width 0.2) (layer "F.Cu") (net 3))
 (segment (start 268.5 89.3) (end 262 89.3) (width 0.2) (layer "F.Cu") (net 3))
 (segment (start 269.801 92.811108) (end 269.801 93.888892) (width 0.2) (layer "F.Cu") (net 3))
 (segment (start 269.801 109.911108) (end 266.289892 106.4) (width 0.2) (layer "F.Cu") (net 3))
 (segment (start 269.801 93.888892) (end 265.839892 97.85) (width 0.2) (layer "F.Cu") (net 3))
 (segment (start 269.801 105.099) (end 268.5 106.4) (width 0.2) (layer "F.Cu") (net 3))
 (segment (start 269.801 99.151) (end 269.801 105.099) (width 0.2) (layer "F.Cu") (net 3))
 (segment (start 262 89.3) (end 266.289892 89.3) (width 0.2) (layer "F.Cu") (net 3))
 (segment (start 182.85 142.882024) (end 182.85 148.45) (width 0.2) (layer "F.Cu") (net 3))
 (segment (start 183.948 105.948) (end 185.5 107.5) (width 0.2) (layer "F.Cu") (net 3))
 (segment (start 268.5 106.4) (end 270 107.9) (width 0.2) (layer "F.Cu") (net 3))
 (segment (start 183.948 95.552) (end 183.948 105.948) (width 0.2) (layer "F.Cu") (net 3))
 (segment (start 262.651 132.43676) (end 261.97676 133.111) (width 0.2) (layer "F.Cu") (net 3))
 (segment (start 268.5 114.95) (end 262 114.95) (width 0.2) (layer "F.Cu") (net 3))
 (segment (start 249.975 142.405) (end 247.539 144.841) (width 0.2) (layer "F.Cu") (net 3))
 (segment (start 221.399 145.741) (end 222.7 144.44) (width 0.2) (layer "F.Cu") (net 3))
 (segment (start 182.948 110.052) (end 182.948 138.679976) (width 0.2) (layer "F.Cu") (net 3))
 (segment (start 269.038892 117.699) (end 261.461108 117.699) (width 0.2) (layer "F.Cu") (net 3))
 (segment (start 182.348976 139.279) (end 181.399 140.228976) (width 0.2) (layer "F.Cu") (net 3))
 (segment (start 251.72924 142.405) (end 249.975 142.405) (width 0.2) (layer "F.Cu") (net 3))
 (segment (start 261.02324 133.111) (end 251.72924 142.405) (width 0.2) (layer "F.Cu") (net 3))
 (segment (start 261.02324 133.111) (end 249.29324 144.841) (width 0.2) (layer "F.Cu") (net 3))
 (segment (start 260.699 122.199) (end 262 123.5) (width 0.2) (layer "F.Cu") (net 3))
 (segment (start 182.948 138.679976) (end 181.399 140.228976) (width 0.2) (layer "F.Cu") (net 3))
 (segment (start 269.801 90.601) (end 269.801 96.549) (width 0.2) (layer "F.Cu") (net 3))
 (segment (start 265.839892 97.85) (end 262 97.85) (width 0.2) (layer "F.Cu") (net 3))
 (segment (start 261.5 129.42) (end 262.651 130.571) (width 0.2) (layer "F.Cu") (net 3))
 (segment (start 181.399 140.228976) (end 181.399 141.431024) (width 0.2) (layer "F.Cu") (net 3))
 (segment (start 182.85 148.45) (end 184.9 150.5) (width 0.2) (layer "F.Cu") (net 3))
 (segment (start 261.5 129.42) (end 269.801 121.119) (width 0.2) (layer "F.Cu") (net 3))
 (segment (start 236.95395 144.841) (end 233.91395 141.801) (width 0.2) (layer "F.Cu") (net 3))
 (segment (start 270 107.9) (end 270 113.45) (width 0.2) (layer "F.Cu") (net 3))
 (segment (start 181.399 141.431024) (end 182.85 142.882024) (width 0.2) (layer "F.Cu") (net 3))
 (segment (start 262.651 130.571) (end 262.651 132.43676) (width 0.2) (layer "F.Cu") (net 3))
 (segment (start 206.229 142.281) (end 207.11 141.4) (width 0.2) (layer "F.Cu") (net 3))
 (segment (start 268.5 106.4) (end 262 106.4) (width 0.2) (layer "F.Cu") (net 3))
 (segment (start 269.801 96.549) (end 268.5 97.85) (width 0.2) (layer "F.Cu") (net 3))
 (segment (start 215.805 130.13) (end 206.656 139.279) (width 0.2) (layer "F.Cu") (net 3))
 (segment (start 247.539 144.841) (end 236.95395 144.841) (width 0.2) (layer "F.Cu") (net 3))
 (segment (start 182.248976 142.281) (end 206.229 142.281) (width 0.2) (layer "F.Cu") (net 3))
 (segment (start 269.801 122.199) (end 269.801 118.461108) (width 0.2) (layer "F.Cu") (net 3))
 (segment (start 185.5 107.5) (end 182.948 110.052) (width 0.2) (layer "F.Cu") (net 3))
 (segment (start 268.5 97.85) (end 269.801 99.151) (width 0.2) (layer "F.Cu") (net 3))
 (segment (start 211.451 145.741) (end 221.399 145.741) (width 0.2) (layer "F.Cu") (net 3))
 (segment (start 266.289892 106.4) (end 262 106.4) (width 0.2) (layer "F.Cu") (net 3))
 (segment (start 232.565 81.87) (end 230.025 81.87) (width 0.2) (layer "F.Cu") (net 3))
 (segment (start 206.656 139.279) (end 182.348976 139.279) (width 0.2) (layer "F.Cu") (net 3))
 (segment (start 268.5 123.5) (end 269.801 122.199) (width 0.2) (layer "F.Cu") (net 3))
 (segment (start 239.995 89.3) (end 232.565 81.87) (width 0.2) (layer "B.Cu") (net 3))
 (segment (start 262 89.3) (end 239.995 89.3) (width 0.2) (layer "B.Cu") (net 3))
 (segment (start 226.1 82.61005) (end 226.1 81.69795) (width 0.2) (layer "F.Cu") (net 2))
 (segment (start 244.164 80.769) (end 245.265 81.87) (width 0.2) (layer "F.Cu") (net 2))
 (segment (start 226.1 81.69795) (end 227.02895 80.769) (width 0.2) (layer "F.Cu") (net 2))
 (segment (start 183.349 88.769) (end 219.94105 88.769) (width 0.2) (layer "F.Cu") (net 2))
 (segment (start 184.5 92.46) (end 183.349 91.309) (width 0.2) (layer "F.Cu") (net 2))
 (segment (start 227.02895 80.769) (end 244.164 80.769) (width 0.2) (layer "F.Cu") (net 2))
 (segment (start 183.349 91.309) (end 183.349 88.769) (width 0.2) (layer "F.Cu") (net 2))
 (segment (start 219.94105 88.769) (end 226.1 82.61005) (width 0.2) (layer "F.Cu") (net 2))
 (segment (start 208.185 130.13) (end 208.185 128.542) (width 0.2) (layer "F.Cu") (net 9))
 (segment (start 266.875992 80.769) (end 249.88895 80.769) (width 0.2) (layer "F.Cu") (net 9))
 (segment (start 261.5 137.04) (end 270.802 127.738) (width 0.2) (layer "F.Cu") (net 9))
 (segment (start 249.244 81.41395) (end 249.244 87.256) (width 0.2) (layer "F.Cu") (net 9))
 (segment (start 208.185 128.542) (end 208.5 128.227) (width 0.2) (layer "F.Cu") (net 9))
 (segment (start 212.668628 122.2) (end 209.2 125.668629) (width 0.2) (layer "F.Cu") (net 9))
 (segment (start 270.802 127.738) (end 270.802 84.695008) (width 0.2) (layer "F.Cu") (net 9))
 (segment (start 249.88895 80.769) (end 249.244 81.41395) (width 0.2) (layer "F.Cu") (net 9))
 (segment (start 214.3 122.2) (end 212.668628 122.2) (width 0.2) (layer "F.Cu") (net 9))
 (segment (start 209.2 125.668629) (end 209.2 127.3) (width 0.2) (layer "F.Cu") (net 9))
 (segment (start 270.802 84.695008) (end 266.875992 80.769) (width 0.2) (layer "F.Cu") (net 9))
 (segment (start 249.244 87.256) (end 214.3 122.2) (width 0.2) (layer "F.Cu") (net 9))
 (segment (start 209.2 127.3) (end 209.075 127.425) (width 0.2) (layer "F.Cu") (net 9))
 (segment (start 268.5 93.35) (end 262 93.35) (width 0.2) (layer "F.Cu") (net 7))
 (segment (start 262 93.35) (end 248.906 106.444) (width 0.2) (layer "F.Cu") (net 7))
 (segment (start 248.26105 131.231) (end 246.366 131.231) (width 0.2) (layer "F.Cu") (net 7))
 (segment (start 248.906 106.444) (end 248.906 130.58605) (width 0.2) (layer "F.Cu") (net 7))
 (segment (start 248.906 130.58605) (end 248.26105 131.231) (width 0.2) (layer "F.Cu") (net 7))
 (segment (start 246.366 131.231) (end 245.265 130.13) (width 0.2) (layer "F.Cu") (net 7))
 (segment (start 185.651 95.47676) (end 185.651 91.071) (width 0.2) (layer "F.Cu") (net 1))
 (segment (start 184.349 103.809) (end 184.349 96.77876) (width 0.2) (layer "F.Cu") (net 1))
 (segment (start 184.349 96.77876) (end 185.651 95.47676) (width 0.2) (layer "F.Cu") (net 1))
 (segment (start 254.865 138.595) (end 261.5 131.96) (width 0.2) (layer "F.Cu") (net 1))
 (segment (start 185.5 104.96) (end 184.349 103.809) (width 0.2) (layer "F.Cu") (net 1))
 (segment (start 219.435 89.92) (end 184.5 89.92) (width 0.2) (layer "F.Cu") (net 1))
 (segment (start 184.7425 89.6775) (end 184.5 89.92) (width 0.2) (layer "F.Cu") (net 1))
 (segment (start 227.485 81.87) (end 219.435 89.92) (width 0.2) (layer "F.Cu") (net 1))
 (segment (start 185.651 91.071) (end 184.5 89.92) (width 0.2) (layer "F.Cu") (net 1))
 (segment (start 249.975 138.595) (end 249.000001 138.595) (width 0.2) (layer "F.Cu") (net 1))
 (segment (start 249.975 138.595) (end 254.865 138.595) (width 0.2) (layer "F.Cu") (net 1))
 (segment (start 237.41 139.69) (end 235.525 139.69) (width 0.2) (layer "F.Cu") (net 15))
 (segment (start 235.525 139.69) (end 225.965 130.13) (width 0.2) (layer "F.Cu") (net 15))
 (segment (start 254.26696 133.072932) (end 251.717 133.072932) (width 0.2) (layer "F.Cu") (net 18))
 (segment (start 246.702 138.087932) (end 246.702 141.074968) (width 0.2) (layer "F.Cu") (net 18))
 (segment (start 251.717 133.072932) (end 246.702 138.087932) (width 0.2) (layer "F.Cu") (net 18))
 (segment (start 268.5 119) (end 262 119) (width 0.2) (layer "F.Cu") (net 18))
 (segment (start 244.009032 141.736) (end 237.645 135.371968) (width 0.2) (layer "F.Cu") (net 18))
 (segment (start 262 119) (end 263.301 120.301) (width 0.2) (layer "F.Cu") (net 18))
 (segment (start 246.040968 141.736) (end 244.009032 141.736) (width 0.2) (layer "F.Cu") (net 18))
 (segment (start 237.645 135.371968) (end 237.645 130.13) (width 0.2) (layer "F.Cu") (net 18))
 (segment (start 263.301 120.301) (end 263.301 124.038892) (width 0.2) (layer "F.Cu") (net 18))
 (segment (start 263.301 124.038892) (end 254.26696 133.072932) (width 0.2) (layer "F.Cu") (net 18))
 (segment (start 246.702 141.074968) (end 246.040968 141.736) (width 0.2) (layer "F.Cu") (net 18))
 (segment (start 240 82.5) (end 240 82) (width 0.2) (layer "F.Cu") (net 26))
 (segment (start 240.185 82.315) (end 240 82.5) (width 0.2) (layer "F.Cu") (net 26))
 (segment (start 240.185 81.87) (end 240.185 82.315) (width 0.2) (layer "F.Cu") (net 26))
 (segment (start 259.66776 140.5) (end 250 140.5) (width 0.2) (layer "B.Cu") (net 26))
 (segment (start 263.301 136.86676) (end 259.66776 140.5) (width 0.2) (layer "B.Cu") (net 26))
 (segment (start 241.814 83.499) (end 258.038892 83.499) (width 0.2) (layer "B.Cu") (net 26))
 (segment (start 240.185 81.87) (end 241.814 83.499) (width 0.2) (layer "B.Cu") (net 26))
 (segment (start 263.301 88.761108) (end 263.301 136.86676) (width 0.2) (layer "B.Cu") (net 26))
 (segment (start 258.038892 83.499) (end 263.301 88.761108) (width 0.2) (layer "B.Cu") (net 26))
 (segment (start 185.5 102.42) (end 185.5 102) (width 0.2) (layer "F.Cu") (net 4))
 (segment (start 242.725 81.87) (end 222.175 102.42) (width 0.2) (layer "F.Cu") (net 4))
 (segment (start 222.175 102.42) (end 185.5 102.42) (width 0.2) (layer "F.Cu") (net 4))
 (segment (start 185.5 102) (end 185.92 102.42) (width 0.2) (layer "F.Cu") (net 4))
 (segment (start 225.54 141.4) (end 227.25 139.69) (width 0.2) (layer "F.Cu") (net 14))
 (segment (start 209.65 141.4) (end 225.54 141.4) (width 0.2) (layer "F.Cu") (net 14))
 (segment (start 225.239892 143.74) (end 227.25 143.74) (width 0.2) (layer "F.Cu") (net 5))
 (segment (start 218.479892 150.5) (end 225.239892 143.74) (width 0.2) (layer "F.Cu") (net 5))
 (segment (start 209.65 150.5) (end 218.479892 150.5) (width 0.2) (layer "F.Cu") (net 5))
 (segment (start 238.746 129.67395) (end 237.29905 128.227) (width 0.2) (layer "F.Cu") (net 19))
 (segment (start 212.45205 132.5) (end 187.04 132.5) (width 0.2) (layer "F.Cu") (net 19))
 (segment (start 237.29905 128.227) (end 216.15095 128.227) (width 0.2) (layer "F.Cu") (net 19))
 (segment (start 214.64505 130.307) (end 212.45205 132.5) (width 0.2) (layer "F.Cu") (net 19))
 (segment (start 216.15095 128.227) (end 214.64505 129.7329) (width 0.2) (layer "F.Cu") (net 19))
 (segment (start 238.746 132.316) (end 238.746 129.67395) (width 0.2) (layer "F.Cu") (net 19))
 (segment (start 214.64505 129.7329) (end 214.64505 130.307) (width 0.2) (layer "F.Cu") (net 19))
 (segment (start 187.04 132.5) (end 184.5 129.96) (width 0.2) (layer "F.Cu") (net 19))
 (segment (start 245.025 138.595) (end 238.746 132.316) (width 0.2) (layer "F.Cu") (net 19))
 (segment (start 184.5 132.5) (end 183.349 131.349) (width 0.2) (layer "F.Cu") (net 20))
 (segment (start 246.301 138.254032) (end 246.301 140.833999) (width 0.2) (layer "F.Cu") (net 20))
 (segment (start 240.665685 127.4) (end 239.9 128.165685) (width 0.2) (layer "F.Cu") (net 20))
 (segment (start 241.286 133.239032) (end 246.301 138.254032) (width 0.2) (layer "F.Cu") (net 20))
 (segment (start 183.349 131.349) (end 183.349 128.809) (width 0.2) (layer "F.Cu") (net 20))
 (segment (start 183.349 128.809) (end 184.332 127.826) (width 0.2) (layer "F.Cu") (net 20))
 (segment (start 216.334314 126.6) (end 244.665685 126.6) (width 0.2) (layer "F.Cu") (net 20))
 (segment (start 244.665685 127.4) (end 240.665685 127.4) (width 0.2) (layer "F.Cu") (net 20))
 (segment (start 244.9 126.834315) (end 244.9 127.165685) (width 0.2) (layer "F.Cu") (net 20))
 (segment (start 184.332 127.826) (end 215.108314 127.826) (width 0.2) (layer "F.Cu") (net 20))
 (segment (start 244.665685 126.6) (end 244.9 126.834315) (width 0.2) (layer "F.Cu") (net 20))
 (segment (start 246.301 140.833999) (end 245.999999 141.135) (width 0.2) (layer "F.Cu") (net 20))
 (segment (start 241.286 129.67395) (end 241.286 133.239032) (width 0.2) (layer "F.Cu") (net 20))
 (segment (start 239.9 128.165685) (end 239.9 128.28795) (width 0.2) (layer "F.Cu") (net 20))
 (segment (start 245.999999 141.135) (end 245.025 141.135) (width 0.2) (layer "F.Cu") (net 20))
 (segment (start 239.9 128.28795) (end 241.286 129.67395) (width 0.2) (layer "F.Cu") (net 20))
 (segment (start 244.9 127.165685) (end 244.665685 127.4) (width 0.2) (layer "F.Cu") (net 20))
 (segment (start 215.108314 127.826) (end 216.334314 126.6) (width 0.2) (layer "F.Cu") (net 20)))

